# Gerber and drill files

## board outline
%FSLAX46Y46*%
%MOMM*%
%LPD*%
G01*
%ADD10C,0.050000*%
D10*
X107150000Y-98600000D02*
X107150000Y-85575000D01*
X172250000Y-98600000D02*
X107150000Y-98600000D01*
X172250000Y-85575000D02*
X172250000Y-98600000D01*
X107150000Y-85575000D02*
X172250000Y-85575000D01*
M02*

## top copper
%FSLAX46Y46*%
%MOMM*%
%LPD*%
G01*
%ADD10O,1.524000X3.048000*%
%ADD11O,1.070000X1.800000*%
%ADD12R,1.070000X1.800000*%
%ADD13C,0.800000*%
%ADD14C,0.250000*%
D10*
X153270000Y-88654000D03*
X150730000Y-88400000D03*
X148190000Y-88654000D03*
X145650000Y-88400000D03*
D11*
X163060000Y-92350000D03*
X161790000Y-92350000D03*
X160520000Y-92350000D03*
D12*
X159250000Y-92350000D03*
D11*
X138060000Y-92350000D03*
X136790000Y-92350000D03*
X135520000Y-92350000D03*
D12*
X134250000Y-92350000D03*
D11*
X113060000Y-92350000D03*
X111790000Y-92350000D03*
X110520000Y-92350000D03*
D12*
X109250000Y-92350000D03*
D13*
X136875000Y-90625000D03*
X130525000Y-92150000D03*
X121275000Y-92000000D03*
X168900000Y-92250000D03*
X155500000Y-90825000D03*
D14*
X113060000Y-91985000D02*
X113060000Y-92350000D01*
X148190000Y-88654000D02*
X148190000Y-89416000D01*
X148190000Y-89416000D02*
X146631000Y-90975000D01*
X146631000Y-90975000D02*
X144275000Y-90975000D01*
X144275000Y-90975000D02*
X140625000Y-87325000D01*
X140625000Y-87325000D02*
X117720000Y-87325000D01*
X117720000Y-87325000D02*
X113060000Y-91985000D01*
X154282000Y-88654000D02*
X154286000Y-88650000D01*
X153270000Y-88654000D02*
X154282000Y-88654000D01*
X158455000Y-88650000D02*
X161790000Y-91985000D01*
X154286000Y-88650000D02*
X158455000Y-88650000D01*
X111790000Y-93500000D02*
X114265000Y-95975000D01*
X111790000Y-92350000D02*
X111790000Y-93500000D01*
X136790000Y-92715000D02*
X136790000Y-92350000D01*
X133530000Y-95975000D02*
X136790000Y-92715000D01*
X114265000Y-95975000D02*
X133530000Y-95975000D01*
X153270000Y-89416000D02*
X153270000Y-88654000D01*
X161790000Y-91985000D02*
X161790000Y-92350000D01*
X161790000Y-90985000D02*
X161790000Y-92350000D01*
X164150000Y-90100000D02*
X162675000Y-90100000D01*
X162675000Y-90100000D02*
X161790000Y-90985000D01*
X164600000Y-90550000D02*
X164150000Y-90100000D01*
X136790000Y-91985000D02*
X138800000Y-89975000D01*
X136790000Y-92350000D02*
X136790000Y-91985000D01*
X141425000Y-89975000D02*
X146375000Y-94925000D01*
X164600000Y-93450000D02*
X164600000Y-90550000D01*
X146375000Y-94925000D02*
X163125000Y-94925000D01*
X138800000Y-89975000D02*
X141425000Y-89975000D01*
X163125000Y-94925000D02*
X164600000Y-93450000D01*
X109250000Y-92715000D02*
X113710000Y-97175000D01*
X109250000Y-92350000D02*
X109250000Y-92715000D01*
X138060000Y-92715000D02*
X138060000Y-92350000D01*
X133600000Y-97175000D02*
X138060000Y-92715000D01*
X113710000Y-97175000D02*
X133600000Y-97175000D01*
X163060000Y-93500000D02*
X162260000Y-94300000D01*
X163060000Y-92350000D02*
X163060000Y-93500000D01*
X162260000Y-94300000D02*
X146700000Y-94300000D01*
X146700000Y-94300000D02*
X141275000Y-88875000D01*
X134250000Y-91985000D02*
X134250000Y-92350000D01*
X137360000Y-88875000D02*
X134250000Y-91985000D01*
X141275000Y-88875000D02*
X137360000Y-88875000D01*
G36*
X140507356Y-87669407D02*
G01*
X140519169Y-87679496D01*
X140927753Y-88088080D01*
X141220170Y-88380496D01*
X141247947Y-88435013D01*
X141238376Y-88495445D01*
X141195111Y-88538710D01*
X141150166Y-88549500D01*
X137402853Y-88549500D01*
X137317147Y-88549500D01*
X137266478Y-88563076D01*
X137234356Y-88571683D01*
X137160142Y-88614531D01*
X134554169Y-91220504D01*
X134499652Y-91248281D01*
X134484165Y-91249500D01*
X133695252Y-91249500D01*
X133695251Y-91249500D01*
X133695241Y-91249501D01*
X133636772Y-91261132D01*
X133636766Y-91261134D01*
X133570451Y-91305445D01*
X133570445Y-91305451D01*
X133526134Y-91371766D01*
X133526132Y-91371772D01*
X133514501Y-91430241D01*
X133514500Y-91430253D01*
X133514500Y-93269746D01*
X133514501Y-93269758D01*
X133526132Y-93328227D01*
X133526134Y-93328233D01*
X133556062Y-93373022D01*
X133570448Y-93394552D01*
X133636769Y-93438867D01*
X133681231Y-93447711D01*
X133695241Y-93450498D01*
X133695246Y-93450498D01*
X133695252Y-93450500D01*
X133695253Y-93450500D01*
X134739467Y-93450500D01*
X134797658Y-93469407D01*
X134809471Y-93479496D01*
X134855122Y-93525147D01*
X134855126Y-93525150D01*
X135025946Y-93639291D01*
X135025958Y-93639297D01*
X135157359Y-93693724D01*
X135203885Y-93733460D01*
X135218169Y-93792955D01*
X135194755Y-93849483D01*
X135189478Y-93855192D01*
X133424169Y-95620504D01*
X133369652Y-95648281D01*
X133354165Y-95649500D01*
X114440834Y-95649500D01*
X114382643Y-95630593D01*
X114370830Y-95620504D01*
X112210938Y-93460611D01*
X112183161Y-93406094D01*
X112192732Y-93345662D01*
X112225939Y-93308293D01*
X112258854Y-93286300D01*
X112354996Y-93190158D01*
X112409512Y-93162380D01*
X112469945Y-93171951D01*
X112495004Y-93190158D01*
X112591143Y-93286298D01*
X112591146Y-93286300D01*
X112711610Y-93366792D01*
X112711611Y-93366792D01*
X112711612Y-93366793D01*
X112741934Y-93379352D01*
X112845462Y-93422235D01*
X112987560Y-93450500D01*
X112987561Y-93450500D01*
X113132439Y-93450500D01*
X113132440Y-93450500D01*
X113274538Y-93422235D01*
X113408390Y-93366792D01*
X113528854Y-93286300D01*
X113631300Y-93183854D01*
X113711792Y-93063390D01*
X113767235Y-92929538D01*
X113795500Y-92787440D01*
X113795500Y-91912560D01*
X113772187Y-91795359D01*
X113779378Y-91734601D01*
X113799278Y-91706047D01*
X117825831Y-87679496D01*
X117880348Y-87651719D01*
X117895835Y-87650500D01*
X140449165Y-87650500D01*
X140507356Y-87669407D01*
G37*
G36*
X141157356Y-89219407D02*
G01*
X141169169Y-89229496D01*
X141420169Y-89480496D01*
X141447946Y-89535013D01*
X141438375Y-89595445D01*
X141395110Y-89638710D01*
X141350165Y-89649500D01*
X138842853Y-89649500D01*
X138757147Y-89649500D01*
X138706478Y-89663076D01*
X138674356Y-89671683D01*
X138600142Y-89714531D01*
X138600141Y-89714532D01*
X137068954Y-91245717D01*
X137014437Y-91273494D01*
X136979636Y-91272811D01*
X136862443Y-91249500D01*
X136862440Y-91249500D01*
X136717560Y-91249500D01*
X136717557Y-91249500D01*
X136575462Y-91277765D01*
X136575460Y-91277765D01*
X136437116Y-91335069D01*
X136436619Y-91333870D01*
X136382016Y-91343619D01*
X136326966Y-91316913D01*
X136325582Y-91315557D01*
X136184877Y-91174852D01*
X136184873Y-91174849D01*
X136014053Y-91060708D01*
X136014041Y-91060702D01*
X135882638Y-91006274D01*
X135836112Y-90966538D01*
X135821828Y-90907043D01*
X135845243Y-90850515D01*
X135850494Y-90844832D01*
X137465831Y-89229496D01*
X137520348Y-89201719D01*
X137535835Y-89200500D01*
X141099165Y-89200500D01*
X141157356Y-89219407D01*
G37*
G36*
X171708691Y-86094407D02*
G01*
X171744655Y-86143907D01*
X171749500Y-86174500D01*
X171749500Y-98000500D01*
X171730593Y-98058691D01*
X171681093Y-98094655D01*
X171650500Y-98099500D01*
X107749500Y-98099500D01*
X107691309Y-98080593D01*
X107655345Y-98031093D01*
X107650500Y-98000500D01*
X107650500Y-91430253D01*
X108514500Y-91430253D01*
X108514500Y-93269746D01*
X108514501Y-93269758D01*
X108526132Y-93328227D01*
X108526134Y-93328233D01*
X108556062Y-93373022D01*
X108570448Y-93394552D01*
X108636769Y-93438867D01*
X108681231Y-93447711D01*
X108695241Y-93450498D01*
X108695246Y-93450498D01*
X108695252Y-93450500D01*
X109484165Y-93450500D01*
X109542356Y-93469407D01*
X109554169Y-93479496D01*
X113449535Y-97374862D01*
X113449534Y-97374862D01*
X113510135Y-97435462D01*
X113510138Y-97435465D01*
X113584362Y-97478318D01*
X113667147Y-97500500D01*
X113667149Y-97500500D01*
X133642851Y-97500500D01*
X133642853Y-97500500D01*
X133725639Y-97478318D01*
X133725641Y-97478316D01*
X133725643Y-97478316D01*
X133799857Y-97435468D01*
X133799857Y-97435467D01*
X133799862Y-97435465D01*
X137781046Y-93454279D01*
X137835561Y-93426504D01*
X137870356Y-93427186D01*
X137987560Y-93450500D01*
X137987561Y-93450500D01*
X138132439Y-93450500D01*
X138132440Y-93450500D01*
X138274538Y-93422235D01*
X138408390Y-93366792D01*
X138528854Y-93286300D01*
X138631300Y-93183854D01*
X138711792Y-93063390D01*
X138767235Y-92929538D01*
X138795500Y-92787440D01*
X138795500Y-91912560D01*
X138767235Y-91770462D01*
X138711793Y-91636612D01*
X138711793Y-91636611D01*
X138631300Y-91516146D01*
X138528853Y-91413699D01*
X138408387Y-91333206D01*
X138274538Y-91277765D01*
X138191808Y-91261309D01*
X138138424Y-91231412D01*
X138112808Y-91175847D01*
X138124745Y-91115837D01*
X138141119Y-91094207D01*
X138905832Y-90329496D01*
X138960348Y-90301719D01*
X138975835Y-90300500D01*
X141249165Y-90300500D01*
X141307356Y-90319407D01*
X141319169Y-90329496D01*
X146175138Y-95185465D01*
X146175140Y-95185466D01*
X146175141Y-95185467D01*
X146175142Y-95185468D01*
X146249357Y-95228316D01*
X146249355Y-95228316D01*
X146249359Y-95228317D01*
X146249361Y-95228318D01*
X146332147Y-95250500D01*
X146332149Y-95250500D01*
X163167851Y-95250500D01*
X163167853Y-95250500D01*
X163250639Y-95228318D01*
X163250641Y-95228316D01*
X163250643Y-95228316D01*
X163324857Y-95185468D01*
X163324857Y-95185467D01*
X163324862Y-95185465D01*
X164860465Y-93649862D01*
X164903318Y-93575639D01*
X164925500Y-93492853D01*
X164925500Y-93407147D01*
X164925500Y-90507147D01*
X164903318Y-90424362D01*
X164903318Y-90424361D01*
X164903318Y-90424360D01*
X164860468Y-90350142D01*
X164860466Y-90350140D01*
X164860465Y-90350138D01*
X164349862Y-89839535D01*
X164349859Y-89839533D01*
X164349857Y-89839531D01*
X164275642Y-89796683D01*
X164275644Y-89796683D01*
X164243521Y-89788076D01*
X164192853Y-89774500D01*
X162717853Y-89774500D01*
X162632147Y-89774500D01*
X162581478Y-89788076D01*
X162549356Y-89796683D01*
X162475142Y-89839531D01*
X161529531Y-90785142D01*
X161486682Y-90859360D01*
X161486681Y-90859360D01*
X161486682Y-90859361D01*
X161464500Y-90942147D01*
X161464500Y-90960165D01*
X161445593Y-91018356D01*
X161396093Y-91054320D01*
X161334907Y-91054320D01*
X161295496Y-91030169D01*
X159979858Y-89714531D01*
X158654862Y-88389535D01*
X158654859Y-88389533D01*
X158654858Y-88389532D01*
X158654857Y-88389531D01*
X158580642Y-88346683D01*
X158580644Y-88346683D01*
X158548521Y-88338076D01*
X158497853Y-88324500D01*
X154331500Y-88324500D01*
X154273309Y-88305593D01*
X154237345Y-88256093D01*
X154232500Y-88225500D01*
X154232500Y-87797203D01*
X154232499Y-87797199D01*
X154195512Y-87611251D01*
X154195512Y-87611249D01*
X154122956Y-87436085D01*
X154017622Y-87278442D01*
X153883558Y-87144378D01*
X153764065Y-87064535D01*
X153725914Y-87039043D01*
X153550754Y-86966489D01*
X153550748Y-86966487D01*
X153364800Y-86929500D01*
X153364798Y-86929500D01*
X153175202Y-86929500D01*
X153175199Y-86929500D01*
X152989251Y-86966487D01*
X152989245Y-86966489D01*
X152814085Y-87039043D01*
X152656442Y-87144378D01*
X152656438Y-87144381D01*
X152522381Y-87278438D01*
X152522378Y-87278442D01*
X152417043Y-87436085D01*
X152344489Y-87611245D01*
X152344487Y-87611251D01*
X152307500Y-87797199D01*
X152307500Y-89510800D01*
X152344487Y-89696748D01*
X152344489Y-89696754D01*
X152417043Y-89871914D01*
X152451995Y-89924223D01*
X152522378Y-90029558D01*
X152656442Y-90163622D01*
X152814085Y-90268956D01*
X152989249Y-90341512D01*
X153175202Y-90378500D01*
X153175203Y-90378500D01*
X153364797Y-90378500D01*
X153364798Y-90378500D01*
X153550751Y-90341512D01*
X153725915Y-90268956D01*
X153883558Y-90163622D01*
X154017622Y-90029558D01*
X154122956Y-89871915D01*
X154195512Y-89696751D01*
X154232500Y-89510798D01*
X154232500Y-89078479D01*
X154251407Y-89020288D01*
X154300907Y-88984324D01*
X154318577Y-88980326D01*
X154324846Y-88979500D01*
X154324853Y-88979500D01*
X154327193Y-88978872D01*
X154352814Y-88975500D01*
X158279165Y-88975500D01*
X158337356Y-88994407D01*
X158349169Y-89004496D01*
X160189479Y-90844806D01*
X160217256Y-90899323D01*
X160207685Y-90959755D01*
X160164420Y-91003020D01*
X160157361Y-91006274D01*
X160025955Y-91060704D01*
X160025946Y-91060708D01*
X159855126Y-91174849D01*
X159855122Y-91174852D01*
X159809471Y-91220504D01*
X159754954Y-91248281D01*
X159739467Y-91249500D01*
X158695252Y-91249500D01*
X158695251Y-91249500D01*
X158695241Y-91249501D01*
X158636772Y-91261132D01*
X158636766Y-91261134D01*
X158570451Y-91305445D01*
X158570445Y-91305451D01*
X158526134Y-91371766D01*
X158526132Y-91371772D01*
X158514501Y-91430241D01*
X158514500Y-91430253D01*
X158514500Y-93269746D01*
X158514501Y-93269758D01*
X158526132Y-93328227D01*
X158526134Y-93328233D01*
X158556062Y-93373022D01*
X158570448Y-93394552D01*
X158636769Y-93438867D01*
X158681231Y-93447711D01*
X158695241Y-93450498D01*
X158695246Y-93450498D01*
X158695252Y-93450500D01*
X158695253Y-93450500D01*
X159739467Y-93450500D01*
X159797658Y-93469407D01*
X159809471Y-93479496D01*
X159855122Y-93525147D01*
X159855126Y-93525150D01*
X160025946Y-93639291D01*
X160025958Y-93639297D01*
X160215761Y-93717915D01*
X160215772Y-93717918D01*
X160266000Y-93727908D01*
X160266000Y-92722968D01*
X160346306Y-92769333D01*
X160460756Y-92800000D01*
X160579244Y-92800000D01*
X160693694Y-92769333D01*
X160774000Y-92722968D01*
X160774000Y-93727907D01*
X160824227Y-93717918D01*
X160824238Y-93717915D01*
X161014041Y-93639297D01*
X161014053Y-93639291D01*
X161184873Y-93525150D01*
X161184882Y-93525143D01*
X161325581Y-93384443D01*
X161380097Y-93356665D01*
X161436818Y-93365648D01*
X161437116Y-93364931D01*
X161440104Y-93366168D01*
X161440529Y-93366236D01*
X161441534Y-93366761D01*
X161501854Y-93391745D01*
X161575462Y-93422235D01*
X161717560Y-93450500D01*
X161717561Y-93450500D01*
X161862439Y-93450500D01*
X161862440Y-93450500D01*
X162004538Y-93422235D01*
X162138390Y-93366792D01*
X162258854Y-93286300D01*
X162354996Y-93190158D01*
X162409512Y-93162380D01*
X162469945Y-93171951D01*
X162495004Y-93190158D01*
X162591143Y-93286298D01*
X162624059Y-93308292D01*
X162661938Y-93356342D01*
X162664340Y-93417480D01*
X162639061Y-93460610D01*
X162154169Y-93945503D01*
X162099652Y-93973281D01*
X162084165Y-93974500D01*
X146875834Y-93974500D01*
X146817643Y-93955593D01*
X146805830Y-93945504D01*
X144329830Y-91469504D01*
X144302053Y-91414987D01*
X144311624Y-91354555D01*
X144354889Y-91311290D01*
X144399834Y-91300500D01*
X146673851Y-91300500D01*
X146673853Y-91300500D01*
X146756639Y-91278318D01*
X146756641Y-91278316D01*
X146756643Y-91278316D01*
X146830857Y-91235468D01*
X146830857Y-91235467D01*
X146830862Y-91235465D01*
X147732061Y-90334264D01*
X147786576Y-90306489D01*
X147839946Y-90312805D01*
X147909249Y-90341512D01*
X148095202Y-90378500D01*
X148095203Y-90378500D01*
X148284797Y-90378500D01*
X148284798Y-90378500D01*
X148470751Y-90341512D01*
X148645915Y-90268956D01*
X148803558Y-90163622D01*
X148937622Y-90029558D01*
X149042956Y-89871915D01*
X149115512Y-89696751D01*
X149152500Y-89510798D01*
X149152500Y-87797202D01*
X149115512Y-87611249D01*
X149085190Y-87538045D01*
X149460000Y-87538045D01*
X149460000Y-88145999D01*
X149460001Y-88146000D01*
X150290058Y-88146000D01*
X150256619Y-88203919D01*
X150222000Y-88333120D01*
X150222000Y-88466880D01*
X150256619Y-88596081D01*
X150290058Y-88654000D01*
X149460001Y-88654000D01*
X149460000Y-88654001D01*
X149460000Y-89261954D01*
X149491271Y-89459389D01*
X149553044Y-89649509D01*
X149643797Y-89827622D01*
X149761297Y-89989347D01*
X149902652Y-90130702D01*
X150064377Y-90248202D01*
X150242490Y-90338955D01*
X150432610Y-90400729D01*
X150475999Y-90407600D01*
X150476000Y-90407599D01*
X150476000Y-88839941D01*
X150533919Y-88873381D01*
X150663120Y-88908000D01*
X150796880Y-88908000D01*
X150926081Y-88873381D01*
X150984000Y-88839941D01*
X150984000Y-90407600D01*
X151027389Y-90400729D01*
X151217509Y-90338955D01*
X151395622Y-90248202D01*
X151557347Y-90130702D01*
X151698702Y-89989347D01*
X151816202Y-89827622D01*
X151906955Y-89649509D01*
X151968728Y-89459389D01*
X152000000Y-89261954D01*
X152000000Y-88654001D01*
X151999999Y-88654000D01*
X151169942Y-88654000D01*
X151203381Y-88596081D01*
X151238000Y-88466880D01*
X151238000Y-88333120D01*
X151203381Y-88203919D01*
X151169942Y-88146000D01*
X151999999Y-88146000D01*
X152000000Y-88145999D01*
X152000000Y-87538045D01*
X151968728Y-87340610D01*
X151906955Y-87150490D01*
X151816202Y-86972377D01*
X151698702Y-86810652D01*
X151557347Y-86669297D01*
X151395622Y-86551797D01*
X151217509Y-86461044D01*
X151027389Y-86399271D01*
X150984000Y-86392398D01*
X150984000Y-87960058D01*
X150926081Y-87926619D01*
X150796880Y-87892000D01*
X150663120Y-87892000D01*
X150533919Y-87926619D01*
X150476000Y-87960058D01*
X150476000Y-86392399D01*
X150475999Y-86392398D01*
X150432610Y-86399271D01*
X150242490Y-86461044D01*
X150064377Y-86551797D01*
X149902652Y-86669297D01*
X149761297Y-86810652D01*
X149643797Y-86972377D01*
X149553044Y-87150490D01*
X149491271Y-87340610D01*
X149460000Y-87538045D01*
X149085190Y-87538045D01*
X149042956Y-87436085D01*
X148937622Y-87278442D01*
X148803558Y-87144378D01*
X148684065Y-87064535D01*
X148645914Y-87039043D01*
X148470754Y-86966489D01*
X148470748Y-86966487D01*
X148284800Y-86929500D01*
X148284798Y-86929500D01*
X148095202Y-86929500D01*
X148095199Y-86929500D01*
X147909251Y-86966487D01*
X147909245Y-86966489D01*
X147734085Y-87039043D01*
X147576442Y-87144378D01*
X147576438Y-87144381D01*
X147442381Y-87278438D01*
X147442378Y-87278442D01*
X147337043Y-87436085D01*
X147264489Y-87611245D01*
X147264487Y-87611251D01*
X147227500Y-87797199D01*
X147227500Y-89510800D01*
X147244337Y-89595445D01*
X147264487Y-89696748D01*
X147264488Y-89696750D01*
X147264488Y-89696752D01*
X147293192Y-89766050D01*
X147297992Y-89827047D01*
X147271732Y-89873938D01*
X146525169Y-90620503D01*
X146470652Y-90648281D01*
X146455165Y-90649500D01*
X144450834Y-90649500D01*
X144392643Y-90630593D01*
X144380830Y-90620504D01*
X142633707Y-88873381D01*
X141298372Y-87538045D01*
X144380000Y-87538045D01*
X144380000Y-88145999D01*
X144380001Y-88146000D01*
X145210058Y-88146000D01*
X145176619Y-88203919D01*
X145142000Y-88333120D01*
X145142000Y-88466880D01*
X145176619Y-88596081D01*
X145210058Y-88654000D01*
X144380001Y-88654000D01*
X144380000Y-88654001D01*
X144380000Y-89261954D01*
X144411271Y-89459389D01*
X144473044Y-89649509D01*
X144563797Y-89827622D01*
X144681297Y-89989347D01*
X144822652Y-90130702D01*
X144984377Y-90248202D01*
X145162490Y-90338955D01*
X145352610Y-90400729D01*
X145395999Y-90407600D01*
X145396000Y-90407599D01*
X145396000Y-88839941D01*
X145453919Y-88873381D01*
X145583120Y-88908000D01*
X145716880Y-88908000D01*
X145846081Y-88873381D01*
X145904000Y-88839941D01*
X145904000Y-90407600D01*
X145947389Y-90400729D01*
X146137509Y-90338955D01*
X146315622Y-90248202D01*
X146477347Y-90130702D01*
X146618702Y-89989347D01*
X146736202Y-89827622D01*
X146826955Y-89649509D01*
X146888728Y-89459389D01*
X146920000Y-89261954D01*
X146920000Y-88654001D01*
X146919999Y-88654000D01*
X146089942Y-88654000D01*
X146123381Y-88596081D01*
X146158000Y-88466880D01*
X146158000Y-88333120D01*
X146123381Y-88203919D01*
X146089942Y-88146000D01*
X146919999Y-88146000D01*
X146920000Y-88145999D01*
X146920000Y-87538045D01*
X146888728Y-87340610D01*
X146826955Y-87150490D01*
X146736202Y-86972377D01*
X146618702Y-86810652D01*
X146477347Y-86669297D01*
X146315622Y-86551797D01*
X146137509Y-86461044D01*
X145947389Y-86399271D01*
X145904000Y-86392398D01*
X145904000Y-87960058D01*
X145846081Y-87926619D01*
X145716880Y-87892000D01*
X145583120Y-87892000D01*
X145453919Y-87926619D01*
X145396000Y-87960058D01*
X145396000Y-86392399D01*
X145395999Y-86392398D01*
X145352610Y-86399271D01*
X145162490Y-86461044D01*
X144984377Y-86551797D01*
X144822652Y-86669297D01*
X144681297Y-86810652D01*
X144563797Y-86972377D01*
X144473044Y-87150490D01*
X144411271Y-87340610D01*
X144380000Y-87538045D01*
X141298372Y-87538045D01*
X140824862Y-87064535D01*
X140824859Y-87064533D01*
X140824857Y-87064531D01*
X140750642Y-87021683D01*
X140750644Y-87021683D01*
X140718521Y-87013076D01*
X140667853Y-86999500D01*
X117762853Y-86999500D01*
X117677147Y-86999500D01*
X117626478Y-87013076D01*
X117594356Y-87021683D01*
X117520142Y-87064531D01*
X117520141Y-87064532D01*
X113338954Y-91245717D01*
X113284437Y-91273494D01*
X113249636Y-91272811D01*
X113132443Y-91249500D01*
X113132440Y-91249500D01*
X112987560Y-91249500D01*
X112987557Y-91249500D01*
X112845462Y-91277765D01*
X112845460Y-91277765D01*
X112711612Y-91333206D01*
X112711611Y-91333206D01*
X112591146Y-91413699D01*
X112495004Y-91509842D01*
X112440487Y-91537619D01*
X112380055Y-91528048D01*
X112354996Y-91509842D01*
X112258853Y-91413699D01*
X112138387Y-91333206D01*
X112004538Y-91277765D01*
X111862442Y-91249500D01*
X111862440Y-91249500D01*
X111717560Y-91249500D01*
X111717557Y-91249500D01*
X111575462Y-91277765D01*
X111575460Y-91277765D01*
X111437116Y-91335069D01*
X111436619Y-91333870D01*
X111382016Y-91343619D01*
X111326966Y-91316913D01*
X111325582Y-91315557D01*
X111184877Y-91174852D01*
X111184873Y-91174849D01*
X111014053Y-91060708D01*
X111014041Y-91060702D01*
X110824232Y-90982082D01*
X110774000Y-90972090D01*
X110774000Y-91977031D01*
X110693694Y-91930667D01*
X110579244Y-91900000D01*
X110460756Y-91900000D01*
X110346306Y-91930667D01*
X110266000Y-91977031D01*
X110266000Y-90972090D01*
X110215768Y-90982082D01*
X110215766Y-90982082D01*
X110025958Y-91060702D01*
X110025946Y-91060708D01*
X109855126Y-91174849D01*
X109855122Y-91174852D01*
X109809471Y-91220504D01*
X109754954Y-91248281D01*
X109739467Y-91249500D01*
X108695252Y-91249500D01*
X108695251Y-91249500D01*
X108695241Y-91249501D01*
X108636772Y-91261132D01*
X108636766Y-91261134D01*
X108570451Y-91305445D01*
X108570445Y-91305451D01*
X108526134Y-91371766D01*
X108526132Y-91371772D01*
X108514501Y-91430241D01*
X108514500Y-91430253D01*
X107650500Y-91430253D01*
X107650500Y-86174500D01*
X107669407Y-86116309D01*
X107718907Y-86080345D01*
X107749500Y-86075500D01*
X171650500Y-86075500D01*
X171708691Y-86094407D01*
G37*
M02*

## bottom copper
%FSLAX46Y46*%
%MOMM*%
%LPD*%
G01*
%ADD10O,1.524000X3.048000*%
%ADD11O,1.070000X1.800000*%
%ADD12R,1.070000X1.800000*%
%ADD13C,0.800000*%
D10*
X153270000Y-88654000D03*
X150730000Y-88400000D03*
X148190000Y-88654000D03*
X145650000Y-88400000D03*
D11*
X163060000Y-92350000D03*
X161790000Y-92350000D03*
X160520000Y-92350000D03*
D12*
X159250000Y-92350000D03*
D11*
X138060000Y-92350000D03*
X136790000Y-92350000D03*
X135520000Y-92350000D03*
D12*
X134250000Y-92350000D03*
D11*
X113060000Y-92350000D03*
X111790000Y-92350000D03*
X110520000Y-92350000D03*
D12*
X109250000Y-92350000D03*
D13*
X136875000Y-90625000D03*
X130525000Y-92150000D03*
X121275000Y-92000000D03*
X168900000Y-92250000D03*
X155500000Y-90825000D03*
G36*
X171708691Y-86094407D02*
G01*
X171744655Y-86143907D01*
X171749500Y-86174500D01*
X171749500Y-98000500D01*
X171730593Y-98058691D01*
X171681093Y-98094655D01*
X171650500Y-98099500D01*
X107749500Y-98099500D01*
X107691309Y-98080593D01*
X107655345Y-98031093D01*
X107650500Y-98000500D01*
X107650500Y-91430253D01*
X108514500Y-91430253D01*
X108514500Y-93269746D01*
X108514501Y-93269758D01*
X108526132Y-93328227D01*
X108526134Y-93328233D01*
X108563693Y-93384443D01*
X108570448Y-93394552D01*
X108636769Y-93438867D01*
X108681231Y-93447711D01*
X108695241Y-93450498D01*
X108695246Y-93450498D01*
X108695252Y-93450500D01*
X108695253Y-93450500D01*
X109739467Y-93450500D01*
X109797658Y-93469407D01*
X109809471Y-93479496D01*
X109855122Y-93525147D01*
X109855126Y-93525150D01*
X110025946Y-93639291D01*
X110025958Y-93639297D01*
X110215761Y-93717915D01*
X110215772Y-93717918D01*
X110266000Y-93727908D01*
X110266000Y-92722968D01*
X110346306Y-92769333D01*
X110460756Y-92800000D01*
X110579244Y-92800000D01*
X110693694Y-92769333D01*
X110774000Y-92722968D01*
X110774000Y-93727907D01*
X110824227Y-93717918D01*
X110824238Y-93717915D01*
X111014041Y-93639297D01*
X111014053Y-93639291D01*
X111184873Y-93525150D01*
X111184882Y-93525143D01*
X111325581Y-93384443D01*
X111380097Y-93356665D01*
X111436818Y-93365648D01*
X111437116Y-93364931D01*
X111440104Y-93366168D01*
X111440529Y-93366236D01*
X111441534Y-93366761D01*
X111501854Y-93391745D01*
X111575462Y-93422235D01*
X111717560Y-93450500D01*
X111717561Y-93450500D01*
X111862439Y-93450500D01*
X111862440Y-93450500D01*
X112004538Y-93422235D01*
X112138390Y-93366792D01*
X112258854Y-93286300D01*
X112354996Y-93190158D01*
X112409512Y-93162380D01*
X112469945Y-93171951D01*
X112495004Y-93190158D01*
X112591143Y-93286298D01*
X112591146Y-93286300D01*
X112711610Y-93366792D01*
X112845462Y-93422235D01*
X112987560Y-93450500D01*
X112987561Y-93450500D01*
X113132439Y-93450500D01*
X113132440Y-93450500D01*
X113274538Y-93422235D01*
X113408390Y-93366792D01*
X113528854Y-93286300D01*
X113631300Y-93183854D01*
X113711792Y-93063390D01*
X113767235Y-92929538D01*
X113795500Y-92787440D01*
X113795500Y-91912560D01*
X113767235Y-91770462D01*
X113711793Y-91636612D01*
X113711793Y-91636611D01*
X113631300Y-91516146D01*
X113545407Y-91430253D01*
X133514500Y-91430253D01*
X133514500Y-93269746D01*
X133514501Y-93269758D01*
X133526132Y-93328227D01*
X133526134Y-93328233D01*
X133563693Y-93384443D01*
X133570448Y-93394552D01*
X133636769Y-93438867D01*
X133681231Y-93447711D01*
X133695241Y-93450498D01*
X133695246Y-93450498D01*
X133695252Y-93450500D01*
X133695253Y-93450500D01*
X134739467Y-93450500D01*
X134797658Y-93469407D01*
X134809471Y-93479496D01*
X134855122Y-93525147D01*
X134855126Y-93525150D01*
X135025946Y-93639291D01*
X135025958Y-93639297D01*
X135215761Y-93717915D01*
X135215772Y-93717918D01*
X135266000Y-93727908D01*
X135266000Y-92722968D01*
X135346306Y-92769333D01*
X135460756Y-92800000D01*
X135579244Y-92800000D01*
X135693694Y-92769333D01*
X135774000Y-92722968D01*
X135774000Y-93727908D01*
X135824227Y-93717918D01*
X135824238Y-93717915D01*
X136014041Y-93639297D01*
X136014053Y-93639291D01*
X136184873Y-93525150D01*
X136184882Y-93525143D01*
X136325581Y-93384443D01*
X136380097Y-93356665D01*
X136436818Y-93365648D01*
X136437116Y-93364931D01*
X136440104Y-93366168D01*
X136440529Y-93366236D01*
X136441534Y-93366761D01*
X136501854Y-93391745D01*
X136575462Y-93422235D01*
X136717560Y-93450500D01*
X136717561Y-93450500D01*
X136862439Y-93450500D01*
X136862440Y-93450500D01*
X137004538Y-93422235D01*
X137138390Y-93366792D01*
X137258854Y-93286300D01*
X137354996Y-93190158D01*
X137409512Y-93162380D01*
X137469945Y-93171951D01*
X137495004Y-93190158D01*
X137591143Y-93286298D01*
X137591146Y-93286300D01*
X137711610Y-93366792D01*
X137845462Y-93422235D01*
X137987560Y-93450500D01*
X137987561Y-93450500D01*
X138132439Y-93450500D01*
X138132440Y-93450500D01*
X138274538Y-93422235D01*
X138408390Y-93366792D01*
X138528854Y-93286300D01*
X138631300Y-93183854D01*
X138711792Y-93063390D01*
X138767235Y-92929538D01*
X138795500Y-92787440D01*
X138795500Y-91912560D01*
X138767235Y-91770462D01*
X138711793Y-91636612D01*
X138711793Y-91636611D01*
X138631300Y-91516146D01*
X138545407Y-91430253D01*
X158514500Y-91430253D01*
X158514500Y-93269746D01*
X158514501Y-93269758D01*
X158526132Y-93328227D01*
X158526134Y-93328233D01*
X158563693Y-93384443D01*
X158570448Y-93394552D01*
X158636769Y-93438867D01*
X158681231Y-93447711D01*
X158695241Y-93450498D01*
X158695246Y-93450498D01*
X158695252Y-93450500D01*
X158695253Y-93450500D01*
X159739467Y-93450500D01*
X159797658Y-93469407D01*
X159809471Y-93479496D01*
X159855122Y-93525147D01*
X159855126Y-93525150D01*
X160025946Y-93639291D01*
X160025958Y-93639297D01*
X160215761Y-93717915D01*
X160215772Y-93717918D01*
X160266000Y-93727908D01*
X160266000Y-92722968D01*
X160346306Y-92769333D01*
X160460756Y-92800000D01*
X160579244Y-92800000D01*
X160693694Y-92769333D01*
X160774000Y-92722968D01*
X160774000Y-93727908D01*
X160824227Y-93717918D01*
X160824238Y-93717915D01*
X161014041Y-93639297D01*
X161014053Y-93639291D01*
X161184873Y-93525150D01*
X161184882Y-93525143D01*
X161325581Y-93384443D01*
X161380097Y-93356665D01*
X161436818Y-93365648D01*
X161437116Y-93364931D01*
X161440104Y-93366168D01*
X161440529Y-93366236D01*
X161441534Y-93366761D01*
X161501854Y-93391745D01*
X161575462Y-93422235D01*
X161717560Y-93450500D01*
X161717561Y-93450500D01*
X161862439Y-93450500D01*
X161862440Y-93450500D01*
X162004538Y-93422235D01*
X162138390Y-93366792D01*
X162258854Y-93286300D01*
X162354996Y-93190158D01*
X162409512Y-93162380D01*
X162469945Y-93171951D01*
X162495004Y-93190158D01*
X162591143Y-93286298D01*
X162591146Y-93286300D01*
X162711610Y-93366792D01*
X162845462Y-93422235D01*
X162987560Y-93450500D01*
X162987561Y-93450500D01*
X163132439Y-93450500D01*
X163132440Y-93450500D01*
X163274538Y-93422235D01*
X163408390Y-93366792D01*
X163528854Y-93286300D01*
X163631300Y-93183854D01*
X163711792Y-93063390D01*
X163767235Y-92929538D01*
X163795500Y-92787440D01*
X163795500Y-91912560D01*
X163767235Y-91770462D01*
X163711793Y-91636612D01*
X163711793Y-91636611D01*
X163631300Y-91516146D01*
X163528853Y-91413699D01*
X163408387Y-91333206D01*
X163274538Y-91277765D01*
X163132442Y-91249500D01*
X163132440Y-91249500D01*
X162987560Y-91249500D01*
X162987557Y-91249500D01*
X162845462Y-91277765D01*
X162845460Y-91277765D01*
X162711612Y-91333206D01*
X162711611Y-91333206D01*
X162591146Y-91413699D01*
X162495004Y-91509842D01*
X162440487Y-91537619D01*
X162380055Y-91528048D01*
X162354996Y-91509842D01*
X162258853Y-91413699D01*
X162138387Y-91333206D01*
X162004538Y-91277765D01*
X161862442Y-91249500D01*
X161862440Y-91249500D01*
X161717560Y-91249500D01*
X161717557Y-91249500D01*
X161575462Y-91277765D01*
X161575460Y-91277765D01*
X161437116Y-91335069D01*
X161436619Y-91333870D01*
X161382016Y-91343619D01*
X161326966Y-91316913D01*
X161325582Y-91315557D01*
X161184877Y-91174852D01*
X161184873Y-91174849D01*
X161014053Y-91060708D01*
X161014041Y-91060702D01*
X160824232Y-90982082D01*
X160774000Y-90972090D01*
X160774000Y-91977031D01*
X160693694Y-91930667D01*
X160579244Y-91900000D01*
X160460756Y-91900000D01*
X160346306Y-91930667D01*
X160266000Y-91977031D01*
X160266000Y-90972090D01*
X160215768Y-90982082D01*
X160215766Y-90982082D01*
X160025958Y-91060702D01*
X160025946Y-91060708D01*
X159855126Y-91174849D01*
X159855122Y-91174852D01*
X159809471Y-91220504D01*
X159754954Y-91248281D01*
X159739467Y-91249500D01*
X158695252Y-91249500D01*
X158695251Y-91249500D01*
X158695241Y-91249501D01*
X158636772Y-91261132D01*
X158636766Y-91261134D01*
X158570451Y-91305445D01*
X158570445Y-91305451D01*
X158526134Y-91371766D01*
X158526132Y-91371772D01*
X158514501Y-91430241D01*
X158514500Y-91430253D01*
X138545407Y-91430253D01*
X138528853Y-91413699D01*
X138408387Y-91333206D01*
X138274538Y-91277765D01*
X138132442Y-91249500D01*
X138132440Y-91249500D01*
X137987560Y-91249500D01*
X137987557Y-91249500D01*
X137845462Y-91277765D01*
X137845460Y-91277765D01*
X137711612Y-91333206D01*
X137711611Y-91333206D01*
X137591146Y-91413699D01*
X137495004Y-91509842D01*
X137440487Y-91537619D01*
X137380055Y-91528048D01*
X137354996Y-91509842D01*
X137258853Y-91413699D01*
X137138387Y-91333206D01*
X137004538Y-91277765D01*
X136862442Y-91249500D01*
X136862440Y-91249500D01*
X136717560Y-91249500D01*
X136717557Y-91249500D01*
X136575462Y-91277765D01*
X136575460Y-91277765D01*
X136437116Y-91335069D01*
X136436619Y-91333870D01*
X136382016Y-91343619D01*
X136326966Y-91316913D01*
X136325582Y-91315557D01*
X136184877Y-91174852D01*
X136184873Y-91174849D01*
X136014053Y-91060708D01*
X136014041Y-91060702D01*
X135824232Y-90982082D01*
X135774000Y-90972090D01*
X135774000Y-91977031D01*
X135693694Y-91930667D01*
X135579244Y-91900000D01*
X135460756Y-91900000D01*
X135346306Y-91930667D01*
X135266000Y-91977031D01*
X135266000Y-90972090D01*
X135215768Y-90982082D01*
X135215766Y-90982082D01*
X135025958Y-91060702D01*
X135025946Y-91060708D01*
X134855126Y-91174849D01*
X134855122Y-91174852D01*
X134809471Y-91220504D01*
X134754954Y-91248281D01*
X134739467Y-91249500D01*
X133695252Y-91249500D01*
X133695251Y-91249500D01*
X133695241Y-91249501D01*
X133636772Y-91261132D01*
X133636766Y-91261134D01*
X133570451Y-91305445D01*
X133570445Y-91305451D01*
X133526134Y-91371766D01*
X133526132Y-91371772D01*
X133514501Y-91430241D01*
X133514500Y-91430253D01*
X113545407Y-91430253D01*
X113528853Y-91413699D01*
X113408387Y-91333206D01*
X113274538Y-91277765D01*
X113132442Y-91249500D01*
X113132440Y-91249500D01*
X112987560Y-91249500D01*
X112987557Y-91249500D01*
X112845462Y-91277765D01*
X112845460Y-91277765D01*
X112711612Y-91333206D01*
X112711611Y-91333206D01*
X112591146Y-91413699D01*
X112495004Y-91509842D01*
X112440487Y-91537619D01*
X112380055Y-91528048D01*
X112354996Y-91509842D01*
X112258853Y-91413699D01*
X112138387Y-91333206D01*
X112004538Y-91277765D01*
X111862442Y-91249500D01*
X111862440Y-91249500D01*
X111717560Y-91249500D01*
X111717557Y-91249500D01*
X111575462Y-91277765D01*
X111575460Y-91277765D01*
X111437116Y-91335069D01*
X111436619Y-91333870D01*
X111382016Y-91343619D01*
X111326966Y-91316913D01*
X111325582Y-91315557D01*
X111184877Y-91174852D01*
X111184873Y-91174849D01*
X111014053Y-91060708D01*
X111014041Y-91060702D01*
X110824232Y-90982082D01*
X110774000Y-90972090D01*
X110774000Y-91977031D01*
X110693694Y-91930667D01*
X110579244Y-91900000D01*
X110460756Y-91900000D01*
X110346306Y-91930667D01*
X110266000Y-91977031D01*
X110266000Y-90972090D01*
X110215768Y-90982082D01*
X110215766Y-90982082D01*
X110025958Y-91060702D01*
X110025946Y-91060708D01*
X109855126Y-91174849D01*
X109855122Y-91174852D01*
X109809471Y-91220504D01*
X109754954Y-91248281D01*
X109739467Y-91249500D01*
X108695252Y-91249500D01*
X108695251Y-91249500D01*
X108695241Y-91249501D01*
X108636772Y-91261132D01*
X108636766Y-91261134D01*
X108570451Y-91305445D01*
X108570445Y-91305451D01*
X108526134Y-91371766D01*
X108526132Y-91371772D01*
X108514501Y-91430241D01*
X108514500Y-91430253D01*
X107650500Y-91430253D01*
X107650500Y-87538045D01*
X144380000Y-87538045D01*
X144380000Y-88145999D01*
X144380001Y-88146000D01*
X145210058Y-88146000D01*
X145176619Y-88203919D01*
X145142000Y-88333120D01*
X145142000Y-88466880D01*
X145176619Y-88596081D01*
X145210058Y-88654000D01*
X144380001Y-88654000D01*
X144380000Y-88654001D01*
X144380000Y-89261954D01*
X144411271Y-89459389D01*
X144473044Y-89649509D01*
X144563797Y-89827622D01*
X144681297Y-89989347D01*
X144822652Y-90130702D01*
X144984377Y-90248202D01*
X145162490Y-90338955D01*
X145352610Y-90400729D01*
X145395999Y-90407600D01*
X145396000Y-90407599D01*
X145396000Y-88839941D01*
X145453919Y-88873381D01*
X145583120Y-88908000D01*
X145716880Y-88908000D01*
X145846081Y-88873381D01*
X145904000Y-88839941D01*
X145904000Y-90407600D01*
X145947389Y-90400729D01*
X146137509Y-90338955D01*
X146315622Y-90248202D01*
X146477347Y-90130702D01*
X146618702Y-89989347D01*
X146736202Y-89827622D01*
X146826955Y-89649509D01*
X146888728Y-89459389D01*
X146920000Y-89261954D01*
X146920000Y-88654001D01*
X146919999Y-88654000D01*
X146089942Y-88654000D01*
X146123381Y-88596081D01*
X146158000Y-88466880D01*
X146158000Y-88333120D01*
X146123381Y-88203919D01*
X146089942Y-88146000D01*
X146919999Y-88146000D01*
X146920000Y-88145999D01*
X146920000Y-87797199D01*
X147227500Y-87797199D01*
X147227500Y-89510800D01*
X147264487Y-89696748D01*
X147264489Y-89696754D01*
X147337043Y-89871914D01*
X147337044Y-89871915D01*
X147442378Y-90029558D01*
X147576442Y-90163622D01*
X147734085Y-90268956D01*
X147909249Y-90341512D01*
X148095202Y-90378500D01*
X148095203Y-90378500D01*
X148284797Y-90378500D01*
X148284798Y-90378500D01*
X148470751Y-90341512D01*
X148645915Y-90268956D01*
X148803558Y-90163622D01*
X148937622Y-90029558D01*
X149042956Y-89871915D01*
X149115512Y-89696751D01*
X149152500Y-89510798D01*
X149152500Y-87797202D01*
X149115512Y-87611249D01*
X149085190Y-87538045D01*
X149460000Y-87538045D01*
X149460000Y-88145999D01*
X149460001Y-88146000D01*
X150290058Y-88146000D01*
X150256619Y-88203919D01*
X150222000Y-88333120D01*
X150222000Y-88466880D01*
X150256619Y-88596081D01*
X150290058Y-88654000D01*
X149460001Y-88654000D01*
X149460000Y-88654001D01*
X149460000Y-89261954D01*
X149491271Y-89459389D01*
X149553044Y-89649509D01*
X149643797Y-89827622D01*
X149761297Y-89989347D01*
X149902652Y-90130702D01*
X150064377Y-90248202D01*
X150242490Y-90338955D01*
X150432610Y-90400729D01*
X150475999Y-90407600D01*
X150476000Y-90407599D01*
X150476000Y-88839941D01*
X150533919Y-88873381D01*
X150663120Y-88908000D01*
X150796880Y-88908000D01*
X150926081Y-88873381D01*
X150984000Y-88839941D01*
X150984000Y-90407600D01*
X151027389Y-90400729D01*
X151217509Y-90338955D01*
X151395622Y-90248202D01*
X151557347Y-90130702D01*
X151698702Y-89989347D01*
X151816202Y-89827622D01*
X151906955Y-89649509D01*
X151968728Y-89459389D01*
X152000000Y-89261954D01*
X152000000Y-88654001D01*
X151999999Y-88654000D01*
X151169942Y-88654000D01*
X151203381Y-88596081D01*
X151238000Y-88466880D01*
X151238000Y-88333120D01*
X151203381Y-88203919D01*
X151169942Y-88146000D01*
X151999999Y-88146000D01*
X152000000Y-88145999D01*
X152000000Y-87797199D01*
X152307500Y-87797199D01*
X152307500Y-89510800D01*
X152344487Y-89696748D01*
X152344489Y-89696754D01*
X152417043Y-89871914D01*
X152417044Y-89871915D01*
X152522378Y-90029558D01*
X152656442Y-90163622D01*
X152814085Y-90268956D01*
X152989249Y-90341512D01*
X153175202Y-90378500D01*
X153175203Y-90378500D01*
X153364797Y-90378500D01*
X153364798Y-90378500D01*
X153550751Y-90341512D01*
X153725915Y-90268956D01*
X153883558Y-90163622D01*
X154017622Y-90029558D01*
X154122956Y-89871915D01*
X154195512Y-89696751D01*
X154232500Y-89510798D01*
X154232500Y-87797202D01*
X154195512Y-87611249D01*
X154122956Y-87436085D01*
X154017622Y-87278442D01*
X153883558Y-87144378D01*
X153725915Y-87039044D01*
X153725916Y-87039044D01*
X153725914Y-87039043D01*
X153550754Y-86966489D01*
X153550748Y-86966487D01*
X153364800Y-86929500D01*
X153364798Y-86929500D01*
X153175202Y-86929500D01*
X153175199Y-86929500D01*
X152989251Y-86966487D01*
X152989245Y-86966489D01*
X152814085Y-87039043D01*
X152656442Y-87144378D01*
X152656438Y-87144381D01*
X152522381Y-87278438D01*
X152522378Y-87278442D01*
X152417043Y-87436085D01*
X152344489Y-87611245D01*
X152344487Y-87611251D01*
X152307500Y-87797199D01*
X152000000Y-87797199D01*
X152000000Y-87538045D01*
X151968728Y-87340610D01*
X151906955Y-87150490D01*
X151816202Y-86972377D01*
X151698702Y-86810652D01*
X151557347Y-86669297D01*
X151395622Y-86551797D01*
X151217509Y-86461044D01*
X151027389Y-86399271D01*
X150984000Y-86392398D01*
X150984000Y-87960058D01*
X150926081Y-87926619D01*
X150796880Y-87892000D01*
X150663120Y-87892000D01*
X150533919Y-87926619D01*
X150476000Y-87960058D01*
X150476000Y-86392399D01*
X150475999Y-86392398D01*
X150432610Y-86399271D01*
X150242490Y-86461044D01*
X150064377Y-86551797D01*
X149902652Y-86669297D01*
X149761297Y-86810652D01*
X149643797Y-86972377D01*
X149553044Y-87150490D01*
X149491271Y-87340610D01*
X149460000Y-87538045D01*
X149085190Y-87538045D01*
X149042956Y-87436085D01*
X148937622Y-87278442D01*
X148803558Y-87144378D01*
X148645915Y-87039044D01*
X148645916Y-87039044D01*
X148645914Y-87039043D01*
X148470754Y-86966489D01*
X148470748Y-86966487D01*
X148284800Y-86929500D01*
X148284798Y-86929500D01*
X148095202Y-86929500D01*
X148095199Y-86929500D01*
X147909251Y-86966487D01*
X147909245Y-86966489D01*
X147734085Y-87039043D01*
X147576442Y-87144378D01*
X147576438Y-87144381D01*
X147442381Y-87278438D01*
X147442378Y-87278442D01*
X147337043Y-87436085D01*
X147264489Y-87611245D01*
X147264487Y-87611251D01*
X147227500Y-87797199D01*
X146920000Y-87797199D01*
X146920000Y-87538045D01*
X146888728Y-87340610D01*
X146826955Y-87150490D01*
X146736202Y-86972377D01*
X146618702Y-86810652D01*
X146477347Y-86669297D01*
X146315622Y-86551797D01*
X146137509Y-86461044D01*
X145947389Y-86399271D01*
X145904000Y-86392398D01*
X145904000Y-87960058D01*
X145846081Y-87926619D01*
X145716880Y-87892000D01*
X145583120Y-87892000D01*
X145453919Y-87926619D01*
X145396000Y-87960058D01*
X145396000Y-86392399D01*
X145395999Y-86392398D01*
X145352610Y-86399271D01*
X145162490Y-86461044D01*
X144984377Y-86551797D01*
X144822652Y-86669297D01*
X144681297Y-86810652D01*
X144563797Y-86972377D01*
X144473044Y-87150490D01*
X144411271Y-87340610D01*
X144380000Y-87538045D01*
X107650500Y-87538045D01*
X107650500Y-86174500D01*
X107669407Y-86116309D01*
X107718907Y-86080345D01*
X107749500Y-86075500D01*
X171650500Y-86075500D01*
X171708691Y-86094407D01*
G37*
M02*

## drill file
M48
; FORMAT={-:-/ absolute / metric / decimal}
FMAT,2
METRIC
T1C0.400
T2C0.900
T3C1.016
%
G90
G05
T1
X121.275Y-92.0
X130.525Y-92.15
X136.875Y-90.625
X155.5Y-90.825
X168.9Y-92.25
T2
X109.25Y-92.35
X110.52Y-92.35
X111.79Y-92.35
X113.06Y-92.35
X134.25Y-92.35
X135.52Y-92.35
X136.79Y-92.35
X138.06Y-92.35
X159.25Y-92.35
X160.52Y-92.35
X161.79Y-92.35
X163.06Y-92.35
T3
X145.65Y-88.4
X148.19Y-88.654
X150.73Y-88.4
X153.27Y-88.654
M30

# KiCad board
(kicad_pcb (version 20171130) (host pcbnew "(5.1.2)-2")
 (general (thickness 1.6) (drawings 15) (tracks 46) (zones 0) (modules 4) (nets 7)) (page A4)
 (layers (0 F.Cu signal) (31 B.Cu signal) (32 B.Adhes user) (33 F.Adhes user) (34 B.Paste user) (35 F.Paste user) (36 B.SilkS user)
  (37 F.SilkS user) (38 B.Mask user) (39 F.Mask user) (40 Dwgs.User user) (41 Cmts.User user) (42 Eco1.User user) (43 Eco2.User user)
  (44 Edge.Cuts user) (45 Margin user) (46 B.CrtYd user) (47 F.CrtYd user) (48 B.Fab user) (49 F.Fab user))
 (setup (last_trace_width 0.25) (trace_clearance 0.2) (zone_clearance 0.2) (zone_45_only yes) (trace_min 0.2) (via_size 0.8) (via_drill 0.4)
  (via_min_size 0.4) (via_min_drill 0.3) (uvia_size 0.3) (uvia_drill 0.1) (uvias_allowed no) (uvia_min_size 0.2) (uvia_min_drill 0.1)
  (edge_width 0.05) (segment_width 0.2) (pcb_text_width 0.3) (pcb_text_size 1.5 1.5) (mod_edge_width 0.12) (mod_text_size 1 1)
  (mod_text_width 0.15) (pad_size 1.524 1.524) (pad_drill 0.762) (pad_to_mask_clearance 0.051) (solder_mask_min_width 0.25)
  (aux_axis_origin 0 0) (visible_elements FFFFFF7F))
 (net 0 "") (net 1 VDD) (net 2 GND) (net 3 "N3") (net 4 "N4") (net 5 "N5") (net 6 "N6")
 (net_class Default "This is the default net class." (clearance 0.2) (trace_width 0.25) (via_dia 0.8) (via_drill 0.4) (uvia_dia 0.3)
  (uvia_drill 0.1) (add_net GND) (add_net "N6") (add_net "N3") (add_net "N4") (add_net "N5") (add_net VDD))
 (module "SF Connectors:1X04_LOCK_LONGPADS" (layer F.Cu) (at 145.65 88.4)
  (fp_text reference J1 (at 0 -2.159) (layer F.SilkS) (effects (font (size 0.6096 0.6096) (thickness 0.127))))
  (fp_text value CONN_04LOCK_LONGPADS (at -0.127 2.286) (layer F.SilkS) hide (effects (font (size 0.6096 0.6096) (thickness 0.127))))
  (pad 4 thru_hole oval (at 7.62 0.254 180) (size 1.524 3.048) (drill 1.016) (layers *.Cu *.Mask) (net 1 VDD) (solder_mask_margin 0.1016))
  (pad 3 thru_hole oval (at 5.08 0 180) (size 1.524 3.048) (drill 1.016) (layers *.Cu *.Mask) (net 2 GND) (solder_mask_margin 0.1016))
  (pad 2 thru_hole oval (at 2.54 0.254 180) (size 1.524 3.048) (drill 1.016) (layers *.Cu *.Mask) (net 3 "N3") (solder_mask_margin 0.1016))
  (pad 1 thru_hole oval (at 0 0 180) (size 1.524 3.048) (drill 1.016) (layers *.Cu *.Mask) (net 2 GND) (solder_mask_margin 0.1016)))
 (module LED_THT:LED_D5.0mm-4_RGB (layer F.Cu) (at 159.25 92.35)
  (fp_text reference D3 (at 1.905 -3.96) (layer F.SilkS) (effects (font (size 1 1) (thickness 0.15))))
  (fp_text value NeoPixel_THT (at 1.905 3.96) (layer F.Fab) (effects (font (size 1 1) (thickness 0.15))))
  (pad 4 thru_hole oval (at 3.81 0) (size 1.07 1.8) (drill 0.9) (layers *.Cu *.Mask) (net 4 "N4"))
  (pad 3 thru_hole oval (at 2.54 0) (size 1.07 1.8) (drill 0.9) (layers *.Cu *.Mask) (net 1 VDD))
  (pad 2 thru_hole oval (at 1.27 0) (size 1.07 1.8) (drill 0.9) (layers *.Cu *.Mask) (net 2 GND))
  (pad 1 thru_hole rect (at 0 0) (size 1.07 1.8) (drill 0.9) (layers *.Cu *.Mask) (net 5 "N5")))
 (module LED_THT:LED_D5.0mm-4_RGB (layer F.Cu) (at 134.25 92.35)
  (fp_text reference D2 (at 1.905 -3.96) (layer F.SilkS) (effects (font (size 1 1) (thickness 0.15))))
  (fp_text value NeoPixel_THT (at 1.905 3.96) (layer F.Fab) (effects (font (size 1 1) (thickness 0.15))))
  (pad 4 thru_hole oval (at 3.81 0) (size 1.07 1.8) (drill 0.9) (layers *.Cu *.Mask) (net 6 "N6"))
  (pad 3 thru_hole oval (at 2.54 0) (size 1.07 1.8) (drill 0.9) (layers *.Cu *.Mask) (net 1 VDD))
  (pad 2 thru_hole oval (at 1.27 0) (size 1.07 1.8) (drill 0.9) (layers *.Cu *.Mask) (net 2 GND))
  (pad 1 thru_hole rect (at 0 0) (size 1.07 1.8) (drill 0.9) (layers *.Cu *.Mask) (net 4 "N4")))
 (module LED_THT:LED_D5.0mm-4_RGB (layer F.Cu) (at 109.25 92.35)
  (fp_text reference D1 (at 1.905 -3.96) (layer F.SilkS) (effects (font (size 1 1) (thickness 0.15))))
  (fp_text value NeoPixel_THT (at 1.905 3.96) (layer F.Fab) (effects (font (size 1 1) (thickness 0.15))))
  (pad 4 thru_hole oval (at 3.81 0) (size 1.07 1.8) (drill 0.9) (layers *.Cu *.Mask) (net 3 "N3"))
  (pad 3 thru_hole oval (at 2.54 0) (size 1.07 1.8) (drill 0.9) (layers *.Cu *.Mask) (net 1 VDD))
  (pad 2 thru_hole oval (at 1.27 0) (size 1.07 1.8) (drill 0.9) (layers *.Cu *.Mask) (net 2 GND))
  (pad 1 thru_hole rect (at 0 0) (size 1.07 1.8) (drill 0.9) (layers *.Cu *.Mask) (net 6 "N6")))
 (gr_line (start 107.15 98.6) (end 107.15 85.575) (layer Edge.Cuts) (width 0.05))
 (gr_line (start 172.25 98.6) (end 107.15 98.6) (layer Edge.Cuts) (width 0.05))
 (gr_line (start 172.25 85.575) (end 172.25 98.6) (layer Edge.Cuts) (width 0.05))
 (gr_line (start 107.15 85.575) (end 172.25 85.575) (layer Edge.Cuts) (width 0.05))
 (via (at 136.875 90.625) (size 0.8) (drill 0.4) (layers F.Cu B.Cu) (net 2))
 (via (at 130.525 92.15) (size 0.8) (drill 0.4) (layers F.Cu B.Cu) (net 2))
 (via (at 121.275 92) (size 0.8) (drill 0.4) (layers F.Cu B.Cu) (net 2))
 (segment (start 113.06 91.985) (end 113.06 92.35) (width 0.25) (layer F.Cu) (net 3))
 (segment (start 148.19 88.654) (end 148.19 89.416) (width 0.25) (layer F.Cu) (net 3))
 (segment (start 148.19 89.416) (end 146.631 90.975) (width 0.25) (layer F.Cu) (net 3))
 (segment (start 146.631 90.975) (end 144.275 90.975) (width 0.25) (layer F.Cu) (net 3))
 (segment (start 144.275 90.975) (end 140.625 87.325) (width 0.25) (layer F.Cu) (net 3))
 (segment (start 140.625 87.325) (end 117.72 87.325) (width 0.25) (layer F.Cu) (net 3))
 (segment (start 117.72 87.325) (end 113.06 91.985) (width 0.25) (layer F.Cu) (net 3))
 (segment (start 154.282 88.654) (end 154.286 88.65) (width 0.25) (layer F.Cu) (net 1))
 (segment (start 153.27 88.654) (end 154.282 88.654) (width 0.25) (layer F.Cu) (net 1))
 (segment (start 158.455 88.65) (end 161.79 91.985) (width 0.25) (layer F.Cu) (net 1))
 (segment (start 154.286 88.65) (end 158.455 88.65) (width 0.25) (layer F.Cu) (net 1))
 (segment (start 111.79 93.5) (end 114.265 95.975) (width 0.25) (layer F.Cu) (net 1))
 (segment (start 111.79 92.35) (end 111.79 93.5) (width 0.25) (layer F.Cu) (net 1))
 (segment (start 136.79 92.715) (end 136.79 92.35) (width 0.25) (layer F.Cu) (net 1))
 (segment (start 133.53 95.975) (end 136.79 92.715) (width 0.25) (layer F.Cu) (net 1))
 (segment (start 114.265 95.975) (end 133.53 95.975) (width 0.25) (layer F.Cu) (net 1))
 (segment (start 153.27 89.416) (end 153.27 88.654) (width 0.25) (layer F.Cu) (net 1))
 (segment (start 161.79 91.985) (end 161.79 92.35) (width 0.25) (layer F.Cu) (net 1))
 (segment (start 161.79 90.985) (end 161.79 92.35) (width 0.25) (layer F.Cu) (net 1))
 (segment (start 164.15 90.1) (end 162.675 90.1) (width 0.25) (layer F.Cu) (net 1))
 (segment (start 162.675 90.1) (end 161.79 90.985) (width 0.25) (layer F.Cu) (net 1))
 (segment (start 164.6 90.55) (end 164.15 90.1) (width 0.25) (layer F.Cu) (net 1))
 (segment (start 136.79 91.985) (end 138.8 89.975) (width 0.25) (layer F.Cu) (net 1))
 (segment (start 136.79 92.35) (end 136.79 91.985) (width 0.25) (layer F.Cu) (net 1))
 (segment (start 141.425 89.975) (end 146.375 94.925) (width 0.25) (layer F.Cu) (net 1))
 (segment (start 164.6 93.45) (end 164.6 90.55) (width 0.25) (layer F.Cu) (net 1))
 (segment (start 146.375 94.925) (end 163.125 94.925) (width 0.25) (layer F.Cu) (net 1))
 (segment (start 138.8 89.975) (end 141.425 89.975) (width 0.25) (layer F.Cu) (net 1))
 (segment (start 163.125 94.925) (end 164.6 93.45) (width 0.25) (layer F.Cu) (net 1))
 (via (at 168.9 92.25) (size 0.8) (drill 0.4) (layers F.Cu B.Cu) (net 2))
 (via (at 155.5 90.825) (size 0.8) (drill 0.4) (layers F.Cu B.Cu) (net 2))
 (segment (start 109.25 92.715) (end 113.71 97.175) (width 0.25) (layer F.Cu) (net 6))
 (segment (start 109.25 92.35) (end 109.25 92.715) (width 0.25) (layer F.Cu) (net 6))
 (segment (start 138.06 92.715) (end 138.06 92.35) (width 0.25) (layer F.Cu) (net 6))
 (segment (start 133.6 97.175) (end 138.06 92.715) (width 0.25) (layer F.Cu) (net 6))
 (segment (start 113.71 97.175) (end 133.6 97.175) (width 0.25) (layer F.Cu) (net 6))
 (segment (start 163.06 93.5) (end 162.26 94.3) (width 0.25) (layer F.Cu) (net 4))
 (segment (start 163.06 92.35) (end 163.06 93.5) (width 0.25) (layer F.Cu) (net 4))
 (segment (start 162.26 94.3) (end 146.7 94.3) (width 0.25) (layer F.Cu) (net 4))
 (segment (start 146.7 94.3) (end 141.275 88.875) (width 0.25) (layer F.Cu) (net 4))
 (segment (start 134.25 91.985) (end 134.25 92.35) (width 0.25) (layer F.Cu) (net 4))
 (segment (start 137.36 88.875) (end 134.25 91.985) (width 0.25) (layer F.Cu) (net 4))
 (segment (start 141.275 88.875) (end 137.36 88.875) (width 0.25) (layer F.Cu) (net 4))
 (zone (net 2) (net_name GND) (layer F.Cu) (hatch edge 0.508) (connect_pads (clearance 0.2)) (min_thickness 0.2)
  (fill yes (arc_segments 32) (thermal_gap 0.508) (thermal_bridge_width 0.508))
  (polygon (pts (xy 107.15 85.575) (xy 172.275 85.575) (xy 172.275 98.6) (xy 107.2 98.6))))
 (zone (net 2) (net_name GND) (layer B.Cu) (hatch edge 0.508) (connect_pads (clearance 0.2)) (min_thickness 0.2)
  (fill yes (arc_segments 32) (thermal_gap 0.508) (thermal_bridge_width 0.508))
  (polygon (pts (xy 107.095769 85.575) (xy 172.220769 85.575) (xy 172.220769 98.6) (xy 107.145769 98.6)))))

